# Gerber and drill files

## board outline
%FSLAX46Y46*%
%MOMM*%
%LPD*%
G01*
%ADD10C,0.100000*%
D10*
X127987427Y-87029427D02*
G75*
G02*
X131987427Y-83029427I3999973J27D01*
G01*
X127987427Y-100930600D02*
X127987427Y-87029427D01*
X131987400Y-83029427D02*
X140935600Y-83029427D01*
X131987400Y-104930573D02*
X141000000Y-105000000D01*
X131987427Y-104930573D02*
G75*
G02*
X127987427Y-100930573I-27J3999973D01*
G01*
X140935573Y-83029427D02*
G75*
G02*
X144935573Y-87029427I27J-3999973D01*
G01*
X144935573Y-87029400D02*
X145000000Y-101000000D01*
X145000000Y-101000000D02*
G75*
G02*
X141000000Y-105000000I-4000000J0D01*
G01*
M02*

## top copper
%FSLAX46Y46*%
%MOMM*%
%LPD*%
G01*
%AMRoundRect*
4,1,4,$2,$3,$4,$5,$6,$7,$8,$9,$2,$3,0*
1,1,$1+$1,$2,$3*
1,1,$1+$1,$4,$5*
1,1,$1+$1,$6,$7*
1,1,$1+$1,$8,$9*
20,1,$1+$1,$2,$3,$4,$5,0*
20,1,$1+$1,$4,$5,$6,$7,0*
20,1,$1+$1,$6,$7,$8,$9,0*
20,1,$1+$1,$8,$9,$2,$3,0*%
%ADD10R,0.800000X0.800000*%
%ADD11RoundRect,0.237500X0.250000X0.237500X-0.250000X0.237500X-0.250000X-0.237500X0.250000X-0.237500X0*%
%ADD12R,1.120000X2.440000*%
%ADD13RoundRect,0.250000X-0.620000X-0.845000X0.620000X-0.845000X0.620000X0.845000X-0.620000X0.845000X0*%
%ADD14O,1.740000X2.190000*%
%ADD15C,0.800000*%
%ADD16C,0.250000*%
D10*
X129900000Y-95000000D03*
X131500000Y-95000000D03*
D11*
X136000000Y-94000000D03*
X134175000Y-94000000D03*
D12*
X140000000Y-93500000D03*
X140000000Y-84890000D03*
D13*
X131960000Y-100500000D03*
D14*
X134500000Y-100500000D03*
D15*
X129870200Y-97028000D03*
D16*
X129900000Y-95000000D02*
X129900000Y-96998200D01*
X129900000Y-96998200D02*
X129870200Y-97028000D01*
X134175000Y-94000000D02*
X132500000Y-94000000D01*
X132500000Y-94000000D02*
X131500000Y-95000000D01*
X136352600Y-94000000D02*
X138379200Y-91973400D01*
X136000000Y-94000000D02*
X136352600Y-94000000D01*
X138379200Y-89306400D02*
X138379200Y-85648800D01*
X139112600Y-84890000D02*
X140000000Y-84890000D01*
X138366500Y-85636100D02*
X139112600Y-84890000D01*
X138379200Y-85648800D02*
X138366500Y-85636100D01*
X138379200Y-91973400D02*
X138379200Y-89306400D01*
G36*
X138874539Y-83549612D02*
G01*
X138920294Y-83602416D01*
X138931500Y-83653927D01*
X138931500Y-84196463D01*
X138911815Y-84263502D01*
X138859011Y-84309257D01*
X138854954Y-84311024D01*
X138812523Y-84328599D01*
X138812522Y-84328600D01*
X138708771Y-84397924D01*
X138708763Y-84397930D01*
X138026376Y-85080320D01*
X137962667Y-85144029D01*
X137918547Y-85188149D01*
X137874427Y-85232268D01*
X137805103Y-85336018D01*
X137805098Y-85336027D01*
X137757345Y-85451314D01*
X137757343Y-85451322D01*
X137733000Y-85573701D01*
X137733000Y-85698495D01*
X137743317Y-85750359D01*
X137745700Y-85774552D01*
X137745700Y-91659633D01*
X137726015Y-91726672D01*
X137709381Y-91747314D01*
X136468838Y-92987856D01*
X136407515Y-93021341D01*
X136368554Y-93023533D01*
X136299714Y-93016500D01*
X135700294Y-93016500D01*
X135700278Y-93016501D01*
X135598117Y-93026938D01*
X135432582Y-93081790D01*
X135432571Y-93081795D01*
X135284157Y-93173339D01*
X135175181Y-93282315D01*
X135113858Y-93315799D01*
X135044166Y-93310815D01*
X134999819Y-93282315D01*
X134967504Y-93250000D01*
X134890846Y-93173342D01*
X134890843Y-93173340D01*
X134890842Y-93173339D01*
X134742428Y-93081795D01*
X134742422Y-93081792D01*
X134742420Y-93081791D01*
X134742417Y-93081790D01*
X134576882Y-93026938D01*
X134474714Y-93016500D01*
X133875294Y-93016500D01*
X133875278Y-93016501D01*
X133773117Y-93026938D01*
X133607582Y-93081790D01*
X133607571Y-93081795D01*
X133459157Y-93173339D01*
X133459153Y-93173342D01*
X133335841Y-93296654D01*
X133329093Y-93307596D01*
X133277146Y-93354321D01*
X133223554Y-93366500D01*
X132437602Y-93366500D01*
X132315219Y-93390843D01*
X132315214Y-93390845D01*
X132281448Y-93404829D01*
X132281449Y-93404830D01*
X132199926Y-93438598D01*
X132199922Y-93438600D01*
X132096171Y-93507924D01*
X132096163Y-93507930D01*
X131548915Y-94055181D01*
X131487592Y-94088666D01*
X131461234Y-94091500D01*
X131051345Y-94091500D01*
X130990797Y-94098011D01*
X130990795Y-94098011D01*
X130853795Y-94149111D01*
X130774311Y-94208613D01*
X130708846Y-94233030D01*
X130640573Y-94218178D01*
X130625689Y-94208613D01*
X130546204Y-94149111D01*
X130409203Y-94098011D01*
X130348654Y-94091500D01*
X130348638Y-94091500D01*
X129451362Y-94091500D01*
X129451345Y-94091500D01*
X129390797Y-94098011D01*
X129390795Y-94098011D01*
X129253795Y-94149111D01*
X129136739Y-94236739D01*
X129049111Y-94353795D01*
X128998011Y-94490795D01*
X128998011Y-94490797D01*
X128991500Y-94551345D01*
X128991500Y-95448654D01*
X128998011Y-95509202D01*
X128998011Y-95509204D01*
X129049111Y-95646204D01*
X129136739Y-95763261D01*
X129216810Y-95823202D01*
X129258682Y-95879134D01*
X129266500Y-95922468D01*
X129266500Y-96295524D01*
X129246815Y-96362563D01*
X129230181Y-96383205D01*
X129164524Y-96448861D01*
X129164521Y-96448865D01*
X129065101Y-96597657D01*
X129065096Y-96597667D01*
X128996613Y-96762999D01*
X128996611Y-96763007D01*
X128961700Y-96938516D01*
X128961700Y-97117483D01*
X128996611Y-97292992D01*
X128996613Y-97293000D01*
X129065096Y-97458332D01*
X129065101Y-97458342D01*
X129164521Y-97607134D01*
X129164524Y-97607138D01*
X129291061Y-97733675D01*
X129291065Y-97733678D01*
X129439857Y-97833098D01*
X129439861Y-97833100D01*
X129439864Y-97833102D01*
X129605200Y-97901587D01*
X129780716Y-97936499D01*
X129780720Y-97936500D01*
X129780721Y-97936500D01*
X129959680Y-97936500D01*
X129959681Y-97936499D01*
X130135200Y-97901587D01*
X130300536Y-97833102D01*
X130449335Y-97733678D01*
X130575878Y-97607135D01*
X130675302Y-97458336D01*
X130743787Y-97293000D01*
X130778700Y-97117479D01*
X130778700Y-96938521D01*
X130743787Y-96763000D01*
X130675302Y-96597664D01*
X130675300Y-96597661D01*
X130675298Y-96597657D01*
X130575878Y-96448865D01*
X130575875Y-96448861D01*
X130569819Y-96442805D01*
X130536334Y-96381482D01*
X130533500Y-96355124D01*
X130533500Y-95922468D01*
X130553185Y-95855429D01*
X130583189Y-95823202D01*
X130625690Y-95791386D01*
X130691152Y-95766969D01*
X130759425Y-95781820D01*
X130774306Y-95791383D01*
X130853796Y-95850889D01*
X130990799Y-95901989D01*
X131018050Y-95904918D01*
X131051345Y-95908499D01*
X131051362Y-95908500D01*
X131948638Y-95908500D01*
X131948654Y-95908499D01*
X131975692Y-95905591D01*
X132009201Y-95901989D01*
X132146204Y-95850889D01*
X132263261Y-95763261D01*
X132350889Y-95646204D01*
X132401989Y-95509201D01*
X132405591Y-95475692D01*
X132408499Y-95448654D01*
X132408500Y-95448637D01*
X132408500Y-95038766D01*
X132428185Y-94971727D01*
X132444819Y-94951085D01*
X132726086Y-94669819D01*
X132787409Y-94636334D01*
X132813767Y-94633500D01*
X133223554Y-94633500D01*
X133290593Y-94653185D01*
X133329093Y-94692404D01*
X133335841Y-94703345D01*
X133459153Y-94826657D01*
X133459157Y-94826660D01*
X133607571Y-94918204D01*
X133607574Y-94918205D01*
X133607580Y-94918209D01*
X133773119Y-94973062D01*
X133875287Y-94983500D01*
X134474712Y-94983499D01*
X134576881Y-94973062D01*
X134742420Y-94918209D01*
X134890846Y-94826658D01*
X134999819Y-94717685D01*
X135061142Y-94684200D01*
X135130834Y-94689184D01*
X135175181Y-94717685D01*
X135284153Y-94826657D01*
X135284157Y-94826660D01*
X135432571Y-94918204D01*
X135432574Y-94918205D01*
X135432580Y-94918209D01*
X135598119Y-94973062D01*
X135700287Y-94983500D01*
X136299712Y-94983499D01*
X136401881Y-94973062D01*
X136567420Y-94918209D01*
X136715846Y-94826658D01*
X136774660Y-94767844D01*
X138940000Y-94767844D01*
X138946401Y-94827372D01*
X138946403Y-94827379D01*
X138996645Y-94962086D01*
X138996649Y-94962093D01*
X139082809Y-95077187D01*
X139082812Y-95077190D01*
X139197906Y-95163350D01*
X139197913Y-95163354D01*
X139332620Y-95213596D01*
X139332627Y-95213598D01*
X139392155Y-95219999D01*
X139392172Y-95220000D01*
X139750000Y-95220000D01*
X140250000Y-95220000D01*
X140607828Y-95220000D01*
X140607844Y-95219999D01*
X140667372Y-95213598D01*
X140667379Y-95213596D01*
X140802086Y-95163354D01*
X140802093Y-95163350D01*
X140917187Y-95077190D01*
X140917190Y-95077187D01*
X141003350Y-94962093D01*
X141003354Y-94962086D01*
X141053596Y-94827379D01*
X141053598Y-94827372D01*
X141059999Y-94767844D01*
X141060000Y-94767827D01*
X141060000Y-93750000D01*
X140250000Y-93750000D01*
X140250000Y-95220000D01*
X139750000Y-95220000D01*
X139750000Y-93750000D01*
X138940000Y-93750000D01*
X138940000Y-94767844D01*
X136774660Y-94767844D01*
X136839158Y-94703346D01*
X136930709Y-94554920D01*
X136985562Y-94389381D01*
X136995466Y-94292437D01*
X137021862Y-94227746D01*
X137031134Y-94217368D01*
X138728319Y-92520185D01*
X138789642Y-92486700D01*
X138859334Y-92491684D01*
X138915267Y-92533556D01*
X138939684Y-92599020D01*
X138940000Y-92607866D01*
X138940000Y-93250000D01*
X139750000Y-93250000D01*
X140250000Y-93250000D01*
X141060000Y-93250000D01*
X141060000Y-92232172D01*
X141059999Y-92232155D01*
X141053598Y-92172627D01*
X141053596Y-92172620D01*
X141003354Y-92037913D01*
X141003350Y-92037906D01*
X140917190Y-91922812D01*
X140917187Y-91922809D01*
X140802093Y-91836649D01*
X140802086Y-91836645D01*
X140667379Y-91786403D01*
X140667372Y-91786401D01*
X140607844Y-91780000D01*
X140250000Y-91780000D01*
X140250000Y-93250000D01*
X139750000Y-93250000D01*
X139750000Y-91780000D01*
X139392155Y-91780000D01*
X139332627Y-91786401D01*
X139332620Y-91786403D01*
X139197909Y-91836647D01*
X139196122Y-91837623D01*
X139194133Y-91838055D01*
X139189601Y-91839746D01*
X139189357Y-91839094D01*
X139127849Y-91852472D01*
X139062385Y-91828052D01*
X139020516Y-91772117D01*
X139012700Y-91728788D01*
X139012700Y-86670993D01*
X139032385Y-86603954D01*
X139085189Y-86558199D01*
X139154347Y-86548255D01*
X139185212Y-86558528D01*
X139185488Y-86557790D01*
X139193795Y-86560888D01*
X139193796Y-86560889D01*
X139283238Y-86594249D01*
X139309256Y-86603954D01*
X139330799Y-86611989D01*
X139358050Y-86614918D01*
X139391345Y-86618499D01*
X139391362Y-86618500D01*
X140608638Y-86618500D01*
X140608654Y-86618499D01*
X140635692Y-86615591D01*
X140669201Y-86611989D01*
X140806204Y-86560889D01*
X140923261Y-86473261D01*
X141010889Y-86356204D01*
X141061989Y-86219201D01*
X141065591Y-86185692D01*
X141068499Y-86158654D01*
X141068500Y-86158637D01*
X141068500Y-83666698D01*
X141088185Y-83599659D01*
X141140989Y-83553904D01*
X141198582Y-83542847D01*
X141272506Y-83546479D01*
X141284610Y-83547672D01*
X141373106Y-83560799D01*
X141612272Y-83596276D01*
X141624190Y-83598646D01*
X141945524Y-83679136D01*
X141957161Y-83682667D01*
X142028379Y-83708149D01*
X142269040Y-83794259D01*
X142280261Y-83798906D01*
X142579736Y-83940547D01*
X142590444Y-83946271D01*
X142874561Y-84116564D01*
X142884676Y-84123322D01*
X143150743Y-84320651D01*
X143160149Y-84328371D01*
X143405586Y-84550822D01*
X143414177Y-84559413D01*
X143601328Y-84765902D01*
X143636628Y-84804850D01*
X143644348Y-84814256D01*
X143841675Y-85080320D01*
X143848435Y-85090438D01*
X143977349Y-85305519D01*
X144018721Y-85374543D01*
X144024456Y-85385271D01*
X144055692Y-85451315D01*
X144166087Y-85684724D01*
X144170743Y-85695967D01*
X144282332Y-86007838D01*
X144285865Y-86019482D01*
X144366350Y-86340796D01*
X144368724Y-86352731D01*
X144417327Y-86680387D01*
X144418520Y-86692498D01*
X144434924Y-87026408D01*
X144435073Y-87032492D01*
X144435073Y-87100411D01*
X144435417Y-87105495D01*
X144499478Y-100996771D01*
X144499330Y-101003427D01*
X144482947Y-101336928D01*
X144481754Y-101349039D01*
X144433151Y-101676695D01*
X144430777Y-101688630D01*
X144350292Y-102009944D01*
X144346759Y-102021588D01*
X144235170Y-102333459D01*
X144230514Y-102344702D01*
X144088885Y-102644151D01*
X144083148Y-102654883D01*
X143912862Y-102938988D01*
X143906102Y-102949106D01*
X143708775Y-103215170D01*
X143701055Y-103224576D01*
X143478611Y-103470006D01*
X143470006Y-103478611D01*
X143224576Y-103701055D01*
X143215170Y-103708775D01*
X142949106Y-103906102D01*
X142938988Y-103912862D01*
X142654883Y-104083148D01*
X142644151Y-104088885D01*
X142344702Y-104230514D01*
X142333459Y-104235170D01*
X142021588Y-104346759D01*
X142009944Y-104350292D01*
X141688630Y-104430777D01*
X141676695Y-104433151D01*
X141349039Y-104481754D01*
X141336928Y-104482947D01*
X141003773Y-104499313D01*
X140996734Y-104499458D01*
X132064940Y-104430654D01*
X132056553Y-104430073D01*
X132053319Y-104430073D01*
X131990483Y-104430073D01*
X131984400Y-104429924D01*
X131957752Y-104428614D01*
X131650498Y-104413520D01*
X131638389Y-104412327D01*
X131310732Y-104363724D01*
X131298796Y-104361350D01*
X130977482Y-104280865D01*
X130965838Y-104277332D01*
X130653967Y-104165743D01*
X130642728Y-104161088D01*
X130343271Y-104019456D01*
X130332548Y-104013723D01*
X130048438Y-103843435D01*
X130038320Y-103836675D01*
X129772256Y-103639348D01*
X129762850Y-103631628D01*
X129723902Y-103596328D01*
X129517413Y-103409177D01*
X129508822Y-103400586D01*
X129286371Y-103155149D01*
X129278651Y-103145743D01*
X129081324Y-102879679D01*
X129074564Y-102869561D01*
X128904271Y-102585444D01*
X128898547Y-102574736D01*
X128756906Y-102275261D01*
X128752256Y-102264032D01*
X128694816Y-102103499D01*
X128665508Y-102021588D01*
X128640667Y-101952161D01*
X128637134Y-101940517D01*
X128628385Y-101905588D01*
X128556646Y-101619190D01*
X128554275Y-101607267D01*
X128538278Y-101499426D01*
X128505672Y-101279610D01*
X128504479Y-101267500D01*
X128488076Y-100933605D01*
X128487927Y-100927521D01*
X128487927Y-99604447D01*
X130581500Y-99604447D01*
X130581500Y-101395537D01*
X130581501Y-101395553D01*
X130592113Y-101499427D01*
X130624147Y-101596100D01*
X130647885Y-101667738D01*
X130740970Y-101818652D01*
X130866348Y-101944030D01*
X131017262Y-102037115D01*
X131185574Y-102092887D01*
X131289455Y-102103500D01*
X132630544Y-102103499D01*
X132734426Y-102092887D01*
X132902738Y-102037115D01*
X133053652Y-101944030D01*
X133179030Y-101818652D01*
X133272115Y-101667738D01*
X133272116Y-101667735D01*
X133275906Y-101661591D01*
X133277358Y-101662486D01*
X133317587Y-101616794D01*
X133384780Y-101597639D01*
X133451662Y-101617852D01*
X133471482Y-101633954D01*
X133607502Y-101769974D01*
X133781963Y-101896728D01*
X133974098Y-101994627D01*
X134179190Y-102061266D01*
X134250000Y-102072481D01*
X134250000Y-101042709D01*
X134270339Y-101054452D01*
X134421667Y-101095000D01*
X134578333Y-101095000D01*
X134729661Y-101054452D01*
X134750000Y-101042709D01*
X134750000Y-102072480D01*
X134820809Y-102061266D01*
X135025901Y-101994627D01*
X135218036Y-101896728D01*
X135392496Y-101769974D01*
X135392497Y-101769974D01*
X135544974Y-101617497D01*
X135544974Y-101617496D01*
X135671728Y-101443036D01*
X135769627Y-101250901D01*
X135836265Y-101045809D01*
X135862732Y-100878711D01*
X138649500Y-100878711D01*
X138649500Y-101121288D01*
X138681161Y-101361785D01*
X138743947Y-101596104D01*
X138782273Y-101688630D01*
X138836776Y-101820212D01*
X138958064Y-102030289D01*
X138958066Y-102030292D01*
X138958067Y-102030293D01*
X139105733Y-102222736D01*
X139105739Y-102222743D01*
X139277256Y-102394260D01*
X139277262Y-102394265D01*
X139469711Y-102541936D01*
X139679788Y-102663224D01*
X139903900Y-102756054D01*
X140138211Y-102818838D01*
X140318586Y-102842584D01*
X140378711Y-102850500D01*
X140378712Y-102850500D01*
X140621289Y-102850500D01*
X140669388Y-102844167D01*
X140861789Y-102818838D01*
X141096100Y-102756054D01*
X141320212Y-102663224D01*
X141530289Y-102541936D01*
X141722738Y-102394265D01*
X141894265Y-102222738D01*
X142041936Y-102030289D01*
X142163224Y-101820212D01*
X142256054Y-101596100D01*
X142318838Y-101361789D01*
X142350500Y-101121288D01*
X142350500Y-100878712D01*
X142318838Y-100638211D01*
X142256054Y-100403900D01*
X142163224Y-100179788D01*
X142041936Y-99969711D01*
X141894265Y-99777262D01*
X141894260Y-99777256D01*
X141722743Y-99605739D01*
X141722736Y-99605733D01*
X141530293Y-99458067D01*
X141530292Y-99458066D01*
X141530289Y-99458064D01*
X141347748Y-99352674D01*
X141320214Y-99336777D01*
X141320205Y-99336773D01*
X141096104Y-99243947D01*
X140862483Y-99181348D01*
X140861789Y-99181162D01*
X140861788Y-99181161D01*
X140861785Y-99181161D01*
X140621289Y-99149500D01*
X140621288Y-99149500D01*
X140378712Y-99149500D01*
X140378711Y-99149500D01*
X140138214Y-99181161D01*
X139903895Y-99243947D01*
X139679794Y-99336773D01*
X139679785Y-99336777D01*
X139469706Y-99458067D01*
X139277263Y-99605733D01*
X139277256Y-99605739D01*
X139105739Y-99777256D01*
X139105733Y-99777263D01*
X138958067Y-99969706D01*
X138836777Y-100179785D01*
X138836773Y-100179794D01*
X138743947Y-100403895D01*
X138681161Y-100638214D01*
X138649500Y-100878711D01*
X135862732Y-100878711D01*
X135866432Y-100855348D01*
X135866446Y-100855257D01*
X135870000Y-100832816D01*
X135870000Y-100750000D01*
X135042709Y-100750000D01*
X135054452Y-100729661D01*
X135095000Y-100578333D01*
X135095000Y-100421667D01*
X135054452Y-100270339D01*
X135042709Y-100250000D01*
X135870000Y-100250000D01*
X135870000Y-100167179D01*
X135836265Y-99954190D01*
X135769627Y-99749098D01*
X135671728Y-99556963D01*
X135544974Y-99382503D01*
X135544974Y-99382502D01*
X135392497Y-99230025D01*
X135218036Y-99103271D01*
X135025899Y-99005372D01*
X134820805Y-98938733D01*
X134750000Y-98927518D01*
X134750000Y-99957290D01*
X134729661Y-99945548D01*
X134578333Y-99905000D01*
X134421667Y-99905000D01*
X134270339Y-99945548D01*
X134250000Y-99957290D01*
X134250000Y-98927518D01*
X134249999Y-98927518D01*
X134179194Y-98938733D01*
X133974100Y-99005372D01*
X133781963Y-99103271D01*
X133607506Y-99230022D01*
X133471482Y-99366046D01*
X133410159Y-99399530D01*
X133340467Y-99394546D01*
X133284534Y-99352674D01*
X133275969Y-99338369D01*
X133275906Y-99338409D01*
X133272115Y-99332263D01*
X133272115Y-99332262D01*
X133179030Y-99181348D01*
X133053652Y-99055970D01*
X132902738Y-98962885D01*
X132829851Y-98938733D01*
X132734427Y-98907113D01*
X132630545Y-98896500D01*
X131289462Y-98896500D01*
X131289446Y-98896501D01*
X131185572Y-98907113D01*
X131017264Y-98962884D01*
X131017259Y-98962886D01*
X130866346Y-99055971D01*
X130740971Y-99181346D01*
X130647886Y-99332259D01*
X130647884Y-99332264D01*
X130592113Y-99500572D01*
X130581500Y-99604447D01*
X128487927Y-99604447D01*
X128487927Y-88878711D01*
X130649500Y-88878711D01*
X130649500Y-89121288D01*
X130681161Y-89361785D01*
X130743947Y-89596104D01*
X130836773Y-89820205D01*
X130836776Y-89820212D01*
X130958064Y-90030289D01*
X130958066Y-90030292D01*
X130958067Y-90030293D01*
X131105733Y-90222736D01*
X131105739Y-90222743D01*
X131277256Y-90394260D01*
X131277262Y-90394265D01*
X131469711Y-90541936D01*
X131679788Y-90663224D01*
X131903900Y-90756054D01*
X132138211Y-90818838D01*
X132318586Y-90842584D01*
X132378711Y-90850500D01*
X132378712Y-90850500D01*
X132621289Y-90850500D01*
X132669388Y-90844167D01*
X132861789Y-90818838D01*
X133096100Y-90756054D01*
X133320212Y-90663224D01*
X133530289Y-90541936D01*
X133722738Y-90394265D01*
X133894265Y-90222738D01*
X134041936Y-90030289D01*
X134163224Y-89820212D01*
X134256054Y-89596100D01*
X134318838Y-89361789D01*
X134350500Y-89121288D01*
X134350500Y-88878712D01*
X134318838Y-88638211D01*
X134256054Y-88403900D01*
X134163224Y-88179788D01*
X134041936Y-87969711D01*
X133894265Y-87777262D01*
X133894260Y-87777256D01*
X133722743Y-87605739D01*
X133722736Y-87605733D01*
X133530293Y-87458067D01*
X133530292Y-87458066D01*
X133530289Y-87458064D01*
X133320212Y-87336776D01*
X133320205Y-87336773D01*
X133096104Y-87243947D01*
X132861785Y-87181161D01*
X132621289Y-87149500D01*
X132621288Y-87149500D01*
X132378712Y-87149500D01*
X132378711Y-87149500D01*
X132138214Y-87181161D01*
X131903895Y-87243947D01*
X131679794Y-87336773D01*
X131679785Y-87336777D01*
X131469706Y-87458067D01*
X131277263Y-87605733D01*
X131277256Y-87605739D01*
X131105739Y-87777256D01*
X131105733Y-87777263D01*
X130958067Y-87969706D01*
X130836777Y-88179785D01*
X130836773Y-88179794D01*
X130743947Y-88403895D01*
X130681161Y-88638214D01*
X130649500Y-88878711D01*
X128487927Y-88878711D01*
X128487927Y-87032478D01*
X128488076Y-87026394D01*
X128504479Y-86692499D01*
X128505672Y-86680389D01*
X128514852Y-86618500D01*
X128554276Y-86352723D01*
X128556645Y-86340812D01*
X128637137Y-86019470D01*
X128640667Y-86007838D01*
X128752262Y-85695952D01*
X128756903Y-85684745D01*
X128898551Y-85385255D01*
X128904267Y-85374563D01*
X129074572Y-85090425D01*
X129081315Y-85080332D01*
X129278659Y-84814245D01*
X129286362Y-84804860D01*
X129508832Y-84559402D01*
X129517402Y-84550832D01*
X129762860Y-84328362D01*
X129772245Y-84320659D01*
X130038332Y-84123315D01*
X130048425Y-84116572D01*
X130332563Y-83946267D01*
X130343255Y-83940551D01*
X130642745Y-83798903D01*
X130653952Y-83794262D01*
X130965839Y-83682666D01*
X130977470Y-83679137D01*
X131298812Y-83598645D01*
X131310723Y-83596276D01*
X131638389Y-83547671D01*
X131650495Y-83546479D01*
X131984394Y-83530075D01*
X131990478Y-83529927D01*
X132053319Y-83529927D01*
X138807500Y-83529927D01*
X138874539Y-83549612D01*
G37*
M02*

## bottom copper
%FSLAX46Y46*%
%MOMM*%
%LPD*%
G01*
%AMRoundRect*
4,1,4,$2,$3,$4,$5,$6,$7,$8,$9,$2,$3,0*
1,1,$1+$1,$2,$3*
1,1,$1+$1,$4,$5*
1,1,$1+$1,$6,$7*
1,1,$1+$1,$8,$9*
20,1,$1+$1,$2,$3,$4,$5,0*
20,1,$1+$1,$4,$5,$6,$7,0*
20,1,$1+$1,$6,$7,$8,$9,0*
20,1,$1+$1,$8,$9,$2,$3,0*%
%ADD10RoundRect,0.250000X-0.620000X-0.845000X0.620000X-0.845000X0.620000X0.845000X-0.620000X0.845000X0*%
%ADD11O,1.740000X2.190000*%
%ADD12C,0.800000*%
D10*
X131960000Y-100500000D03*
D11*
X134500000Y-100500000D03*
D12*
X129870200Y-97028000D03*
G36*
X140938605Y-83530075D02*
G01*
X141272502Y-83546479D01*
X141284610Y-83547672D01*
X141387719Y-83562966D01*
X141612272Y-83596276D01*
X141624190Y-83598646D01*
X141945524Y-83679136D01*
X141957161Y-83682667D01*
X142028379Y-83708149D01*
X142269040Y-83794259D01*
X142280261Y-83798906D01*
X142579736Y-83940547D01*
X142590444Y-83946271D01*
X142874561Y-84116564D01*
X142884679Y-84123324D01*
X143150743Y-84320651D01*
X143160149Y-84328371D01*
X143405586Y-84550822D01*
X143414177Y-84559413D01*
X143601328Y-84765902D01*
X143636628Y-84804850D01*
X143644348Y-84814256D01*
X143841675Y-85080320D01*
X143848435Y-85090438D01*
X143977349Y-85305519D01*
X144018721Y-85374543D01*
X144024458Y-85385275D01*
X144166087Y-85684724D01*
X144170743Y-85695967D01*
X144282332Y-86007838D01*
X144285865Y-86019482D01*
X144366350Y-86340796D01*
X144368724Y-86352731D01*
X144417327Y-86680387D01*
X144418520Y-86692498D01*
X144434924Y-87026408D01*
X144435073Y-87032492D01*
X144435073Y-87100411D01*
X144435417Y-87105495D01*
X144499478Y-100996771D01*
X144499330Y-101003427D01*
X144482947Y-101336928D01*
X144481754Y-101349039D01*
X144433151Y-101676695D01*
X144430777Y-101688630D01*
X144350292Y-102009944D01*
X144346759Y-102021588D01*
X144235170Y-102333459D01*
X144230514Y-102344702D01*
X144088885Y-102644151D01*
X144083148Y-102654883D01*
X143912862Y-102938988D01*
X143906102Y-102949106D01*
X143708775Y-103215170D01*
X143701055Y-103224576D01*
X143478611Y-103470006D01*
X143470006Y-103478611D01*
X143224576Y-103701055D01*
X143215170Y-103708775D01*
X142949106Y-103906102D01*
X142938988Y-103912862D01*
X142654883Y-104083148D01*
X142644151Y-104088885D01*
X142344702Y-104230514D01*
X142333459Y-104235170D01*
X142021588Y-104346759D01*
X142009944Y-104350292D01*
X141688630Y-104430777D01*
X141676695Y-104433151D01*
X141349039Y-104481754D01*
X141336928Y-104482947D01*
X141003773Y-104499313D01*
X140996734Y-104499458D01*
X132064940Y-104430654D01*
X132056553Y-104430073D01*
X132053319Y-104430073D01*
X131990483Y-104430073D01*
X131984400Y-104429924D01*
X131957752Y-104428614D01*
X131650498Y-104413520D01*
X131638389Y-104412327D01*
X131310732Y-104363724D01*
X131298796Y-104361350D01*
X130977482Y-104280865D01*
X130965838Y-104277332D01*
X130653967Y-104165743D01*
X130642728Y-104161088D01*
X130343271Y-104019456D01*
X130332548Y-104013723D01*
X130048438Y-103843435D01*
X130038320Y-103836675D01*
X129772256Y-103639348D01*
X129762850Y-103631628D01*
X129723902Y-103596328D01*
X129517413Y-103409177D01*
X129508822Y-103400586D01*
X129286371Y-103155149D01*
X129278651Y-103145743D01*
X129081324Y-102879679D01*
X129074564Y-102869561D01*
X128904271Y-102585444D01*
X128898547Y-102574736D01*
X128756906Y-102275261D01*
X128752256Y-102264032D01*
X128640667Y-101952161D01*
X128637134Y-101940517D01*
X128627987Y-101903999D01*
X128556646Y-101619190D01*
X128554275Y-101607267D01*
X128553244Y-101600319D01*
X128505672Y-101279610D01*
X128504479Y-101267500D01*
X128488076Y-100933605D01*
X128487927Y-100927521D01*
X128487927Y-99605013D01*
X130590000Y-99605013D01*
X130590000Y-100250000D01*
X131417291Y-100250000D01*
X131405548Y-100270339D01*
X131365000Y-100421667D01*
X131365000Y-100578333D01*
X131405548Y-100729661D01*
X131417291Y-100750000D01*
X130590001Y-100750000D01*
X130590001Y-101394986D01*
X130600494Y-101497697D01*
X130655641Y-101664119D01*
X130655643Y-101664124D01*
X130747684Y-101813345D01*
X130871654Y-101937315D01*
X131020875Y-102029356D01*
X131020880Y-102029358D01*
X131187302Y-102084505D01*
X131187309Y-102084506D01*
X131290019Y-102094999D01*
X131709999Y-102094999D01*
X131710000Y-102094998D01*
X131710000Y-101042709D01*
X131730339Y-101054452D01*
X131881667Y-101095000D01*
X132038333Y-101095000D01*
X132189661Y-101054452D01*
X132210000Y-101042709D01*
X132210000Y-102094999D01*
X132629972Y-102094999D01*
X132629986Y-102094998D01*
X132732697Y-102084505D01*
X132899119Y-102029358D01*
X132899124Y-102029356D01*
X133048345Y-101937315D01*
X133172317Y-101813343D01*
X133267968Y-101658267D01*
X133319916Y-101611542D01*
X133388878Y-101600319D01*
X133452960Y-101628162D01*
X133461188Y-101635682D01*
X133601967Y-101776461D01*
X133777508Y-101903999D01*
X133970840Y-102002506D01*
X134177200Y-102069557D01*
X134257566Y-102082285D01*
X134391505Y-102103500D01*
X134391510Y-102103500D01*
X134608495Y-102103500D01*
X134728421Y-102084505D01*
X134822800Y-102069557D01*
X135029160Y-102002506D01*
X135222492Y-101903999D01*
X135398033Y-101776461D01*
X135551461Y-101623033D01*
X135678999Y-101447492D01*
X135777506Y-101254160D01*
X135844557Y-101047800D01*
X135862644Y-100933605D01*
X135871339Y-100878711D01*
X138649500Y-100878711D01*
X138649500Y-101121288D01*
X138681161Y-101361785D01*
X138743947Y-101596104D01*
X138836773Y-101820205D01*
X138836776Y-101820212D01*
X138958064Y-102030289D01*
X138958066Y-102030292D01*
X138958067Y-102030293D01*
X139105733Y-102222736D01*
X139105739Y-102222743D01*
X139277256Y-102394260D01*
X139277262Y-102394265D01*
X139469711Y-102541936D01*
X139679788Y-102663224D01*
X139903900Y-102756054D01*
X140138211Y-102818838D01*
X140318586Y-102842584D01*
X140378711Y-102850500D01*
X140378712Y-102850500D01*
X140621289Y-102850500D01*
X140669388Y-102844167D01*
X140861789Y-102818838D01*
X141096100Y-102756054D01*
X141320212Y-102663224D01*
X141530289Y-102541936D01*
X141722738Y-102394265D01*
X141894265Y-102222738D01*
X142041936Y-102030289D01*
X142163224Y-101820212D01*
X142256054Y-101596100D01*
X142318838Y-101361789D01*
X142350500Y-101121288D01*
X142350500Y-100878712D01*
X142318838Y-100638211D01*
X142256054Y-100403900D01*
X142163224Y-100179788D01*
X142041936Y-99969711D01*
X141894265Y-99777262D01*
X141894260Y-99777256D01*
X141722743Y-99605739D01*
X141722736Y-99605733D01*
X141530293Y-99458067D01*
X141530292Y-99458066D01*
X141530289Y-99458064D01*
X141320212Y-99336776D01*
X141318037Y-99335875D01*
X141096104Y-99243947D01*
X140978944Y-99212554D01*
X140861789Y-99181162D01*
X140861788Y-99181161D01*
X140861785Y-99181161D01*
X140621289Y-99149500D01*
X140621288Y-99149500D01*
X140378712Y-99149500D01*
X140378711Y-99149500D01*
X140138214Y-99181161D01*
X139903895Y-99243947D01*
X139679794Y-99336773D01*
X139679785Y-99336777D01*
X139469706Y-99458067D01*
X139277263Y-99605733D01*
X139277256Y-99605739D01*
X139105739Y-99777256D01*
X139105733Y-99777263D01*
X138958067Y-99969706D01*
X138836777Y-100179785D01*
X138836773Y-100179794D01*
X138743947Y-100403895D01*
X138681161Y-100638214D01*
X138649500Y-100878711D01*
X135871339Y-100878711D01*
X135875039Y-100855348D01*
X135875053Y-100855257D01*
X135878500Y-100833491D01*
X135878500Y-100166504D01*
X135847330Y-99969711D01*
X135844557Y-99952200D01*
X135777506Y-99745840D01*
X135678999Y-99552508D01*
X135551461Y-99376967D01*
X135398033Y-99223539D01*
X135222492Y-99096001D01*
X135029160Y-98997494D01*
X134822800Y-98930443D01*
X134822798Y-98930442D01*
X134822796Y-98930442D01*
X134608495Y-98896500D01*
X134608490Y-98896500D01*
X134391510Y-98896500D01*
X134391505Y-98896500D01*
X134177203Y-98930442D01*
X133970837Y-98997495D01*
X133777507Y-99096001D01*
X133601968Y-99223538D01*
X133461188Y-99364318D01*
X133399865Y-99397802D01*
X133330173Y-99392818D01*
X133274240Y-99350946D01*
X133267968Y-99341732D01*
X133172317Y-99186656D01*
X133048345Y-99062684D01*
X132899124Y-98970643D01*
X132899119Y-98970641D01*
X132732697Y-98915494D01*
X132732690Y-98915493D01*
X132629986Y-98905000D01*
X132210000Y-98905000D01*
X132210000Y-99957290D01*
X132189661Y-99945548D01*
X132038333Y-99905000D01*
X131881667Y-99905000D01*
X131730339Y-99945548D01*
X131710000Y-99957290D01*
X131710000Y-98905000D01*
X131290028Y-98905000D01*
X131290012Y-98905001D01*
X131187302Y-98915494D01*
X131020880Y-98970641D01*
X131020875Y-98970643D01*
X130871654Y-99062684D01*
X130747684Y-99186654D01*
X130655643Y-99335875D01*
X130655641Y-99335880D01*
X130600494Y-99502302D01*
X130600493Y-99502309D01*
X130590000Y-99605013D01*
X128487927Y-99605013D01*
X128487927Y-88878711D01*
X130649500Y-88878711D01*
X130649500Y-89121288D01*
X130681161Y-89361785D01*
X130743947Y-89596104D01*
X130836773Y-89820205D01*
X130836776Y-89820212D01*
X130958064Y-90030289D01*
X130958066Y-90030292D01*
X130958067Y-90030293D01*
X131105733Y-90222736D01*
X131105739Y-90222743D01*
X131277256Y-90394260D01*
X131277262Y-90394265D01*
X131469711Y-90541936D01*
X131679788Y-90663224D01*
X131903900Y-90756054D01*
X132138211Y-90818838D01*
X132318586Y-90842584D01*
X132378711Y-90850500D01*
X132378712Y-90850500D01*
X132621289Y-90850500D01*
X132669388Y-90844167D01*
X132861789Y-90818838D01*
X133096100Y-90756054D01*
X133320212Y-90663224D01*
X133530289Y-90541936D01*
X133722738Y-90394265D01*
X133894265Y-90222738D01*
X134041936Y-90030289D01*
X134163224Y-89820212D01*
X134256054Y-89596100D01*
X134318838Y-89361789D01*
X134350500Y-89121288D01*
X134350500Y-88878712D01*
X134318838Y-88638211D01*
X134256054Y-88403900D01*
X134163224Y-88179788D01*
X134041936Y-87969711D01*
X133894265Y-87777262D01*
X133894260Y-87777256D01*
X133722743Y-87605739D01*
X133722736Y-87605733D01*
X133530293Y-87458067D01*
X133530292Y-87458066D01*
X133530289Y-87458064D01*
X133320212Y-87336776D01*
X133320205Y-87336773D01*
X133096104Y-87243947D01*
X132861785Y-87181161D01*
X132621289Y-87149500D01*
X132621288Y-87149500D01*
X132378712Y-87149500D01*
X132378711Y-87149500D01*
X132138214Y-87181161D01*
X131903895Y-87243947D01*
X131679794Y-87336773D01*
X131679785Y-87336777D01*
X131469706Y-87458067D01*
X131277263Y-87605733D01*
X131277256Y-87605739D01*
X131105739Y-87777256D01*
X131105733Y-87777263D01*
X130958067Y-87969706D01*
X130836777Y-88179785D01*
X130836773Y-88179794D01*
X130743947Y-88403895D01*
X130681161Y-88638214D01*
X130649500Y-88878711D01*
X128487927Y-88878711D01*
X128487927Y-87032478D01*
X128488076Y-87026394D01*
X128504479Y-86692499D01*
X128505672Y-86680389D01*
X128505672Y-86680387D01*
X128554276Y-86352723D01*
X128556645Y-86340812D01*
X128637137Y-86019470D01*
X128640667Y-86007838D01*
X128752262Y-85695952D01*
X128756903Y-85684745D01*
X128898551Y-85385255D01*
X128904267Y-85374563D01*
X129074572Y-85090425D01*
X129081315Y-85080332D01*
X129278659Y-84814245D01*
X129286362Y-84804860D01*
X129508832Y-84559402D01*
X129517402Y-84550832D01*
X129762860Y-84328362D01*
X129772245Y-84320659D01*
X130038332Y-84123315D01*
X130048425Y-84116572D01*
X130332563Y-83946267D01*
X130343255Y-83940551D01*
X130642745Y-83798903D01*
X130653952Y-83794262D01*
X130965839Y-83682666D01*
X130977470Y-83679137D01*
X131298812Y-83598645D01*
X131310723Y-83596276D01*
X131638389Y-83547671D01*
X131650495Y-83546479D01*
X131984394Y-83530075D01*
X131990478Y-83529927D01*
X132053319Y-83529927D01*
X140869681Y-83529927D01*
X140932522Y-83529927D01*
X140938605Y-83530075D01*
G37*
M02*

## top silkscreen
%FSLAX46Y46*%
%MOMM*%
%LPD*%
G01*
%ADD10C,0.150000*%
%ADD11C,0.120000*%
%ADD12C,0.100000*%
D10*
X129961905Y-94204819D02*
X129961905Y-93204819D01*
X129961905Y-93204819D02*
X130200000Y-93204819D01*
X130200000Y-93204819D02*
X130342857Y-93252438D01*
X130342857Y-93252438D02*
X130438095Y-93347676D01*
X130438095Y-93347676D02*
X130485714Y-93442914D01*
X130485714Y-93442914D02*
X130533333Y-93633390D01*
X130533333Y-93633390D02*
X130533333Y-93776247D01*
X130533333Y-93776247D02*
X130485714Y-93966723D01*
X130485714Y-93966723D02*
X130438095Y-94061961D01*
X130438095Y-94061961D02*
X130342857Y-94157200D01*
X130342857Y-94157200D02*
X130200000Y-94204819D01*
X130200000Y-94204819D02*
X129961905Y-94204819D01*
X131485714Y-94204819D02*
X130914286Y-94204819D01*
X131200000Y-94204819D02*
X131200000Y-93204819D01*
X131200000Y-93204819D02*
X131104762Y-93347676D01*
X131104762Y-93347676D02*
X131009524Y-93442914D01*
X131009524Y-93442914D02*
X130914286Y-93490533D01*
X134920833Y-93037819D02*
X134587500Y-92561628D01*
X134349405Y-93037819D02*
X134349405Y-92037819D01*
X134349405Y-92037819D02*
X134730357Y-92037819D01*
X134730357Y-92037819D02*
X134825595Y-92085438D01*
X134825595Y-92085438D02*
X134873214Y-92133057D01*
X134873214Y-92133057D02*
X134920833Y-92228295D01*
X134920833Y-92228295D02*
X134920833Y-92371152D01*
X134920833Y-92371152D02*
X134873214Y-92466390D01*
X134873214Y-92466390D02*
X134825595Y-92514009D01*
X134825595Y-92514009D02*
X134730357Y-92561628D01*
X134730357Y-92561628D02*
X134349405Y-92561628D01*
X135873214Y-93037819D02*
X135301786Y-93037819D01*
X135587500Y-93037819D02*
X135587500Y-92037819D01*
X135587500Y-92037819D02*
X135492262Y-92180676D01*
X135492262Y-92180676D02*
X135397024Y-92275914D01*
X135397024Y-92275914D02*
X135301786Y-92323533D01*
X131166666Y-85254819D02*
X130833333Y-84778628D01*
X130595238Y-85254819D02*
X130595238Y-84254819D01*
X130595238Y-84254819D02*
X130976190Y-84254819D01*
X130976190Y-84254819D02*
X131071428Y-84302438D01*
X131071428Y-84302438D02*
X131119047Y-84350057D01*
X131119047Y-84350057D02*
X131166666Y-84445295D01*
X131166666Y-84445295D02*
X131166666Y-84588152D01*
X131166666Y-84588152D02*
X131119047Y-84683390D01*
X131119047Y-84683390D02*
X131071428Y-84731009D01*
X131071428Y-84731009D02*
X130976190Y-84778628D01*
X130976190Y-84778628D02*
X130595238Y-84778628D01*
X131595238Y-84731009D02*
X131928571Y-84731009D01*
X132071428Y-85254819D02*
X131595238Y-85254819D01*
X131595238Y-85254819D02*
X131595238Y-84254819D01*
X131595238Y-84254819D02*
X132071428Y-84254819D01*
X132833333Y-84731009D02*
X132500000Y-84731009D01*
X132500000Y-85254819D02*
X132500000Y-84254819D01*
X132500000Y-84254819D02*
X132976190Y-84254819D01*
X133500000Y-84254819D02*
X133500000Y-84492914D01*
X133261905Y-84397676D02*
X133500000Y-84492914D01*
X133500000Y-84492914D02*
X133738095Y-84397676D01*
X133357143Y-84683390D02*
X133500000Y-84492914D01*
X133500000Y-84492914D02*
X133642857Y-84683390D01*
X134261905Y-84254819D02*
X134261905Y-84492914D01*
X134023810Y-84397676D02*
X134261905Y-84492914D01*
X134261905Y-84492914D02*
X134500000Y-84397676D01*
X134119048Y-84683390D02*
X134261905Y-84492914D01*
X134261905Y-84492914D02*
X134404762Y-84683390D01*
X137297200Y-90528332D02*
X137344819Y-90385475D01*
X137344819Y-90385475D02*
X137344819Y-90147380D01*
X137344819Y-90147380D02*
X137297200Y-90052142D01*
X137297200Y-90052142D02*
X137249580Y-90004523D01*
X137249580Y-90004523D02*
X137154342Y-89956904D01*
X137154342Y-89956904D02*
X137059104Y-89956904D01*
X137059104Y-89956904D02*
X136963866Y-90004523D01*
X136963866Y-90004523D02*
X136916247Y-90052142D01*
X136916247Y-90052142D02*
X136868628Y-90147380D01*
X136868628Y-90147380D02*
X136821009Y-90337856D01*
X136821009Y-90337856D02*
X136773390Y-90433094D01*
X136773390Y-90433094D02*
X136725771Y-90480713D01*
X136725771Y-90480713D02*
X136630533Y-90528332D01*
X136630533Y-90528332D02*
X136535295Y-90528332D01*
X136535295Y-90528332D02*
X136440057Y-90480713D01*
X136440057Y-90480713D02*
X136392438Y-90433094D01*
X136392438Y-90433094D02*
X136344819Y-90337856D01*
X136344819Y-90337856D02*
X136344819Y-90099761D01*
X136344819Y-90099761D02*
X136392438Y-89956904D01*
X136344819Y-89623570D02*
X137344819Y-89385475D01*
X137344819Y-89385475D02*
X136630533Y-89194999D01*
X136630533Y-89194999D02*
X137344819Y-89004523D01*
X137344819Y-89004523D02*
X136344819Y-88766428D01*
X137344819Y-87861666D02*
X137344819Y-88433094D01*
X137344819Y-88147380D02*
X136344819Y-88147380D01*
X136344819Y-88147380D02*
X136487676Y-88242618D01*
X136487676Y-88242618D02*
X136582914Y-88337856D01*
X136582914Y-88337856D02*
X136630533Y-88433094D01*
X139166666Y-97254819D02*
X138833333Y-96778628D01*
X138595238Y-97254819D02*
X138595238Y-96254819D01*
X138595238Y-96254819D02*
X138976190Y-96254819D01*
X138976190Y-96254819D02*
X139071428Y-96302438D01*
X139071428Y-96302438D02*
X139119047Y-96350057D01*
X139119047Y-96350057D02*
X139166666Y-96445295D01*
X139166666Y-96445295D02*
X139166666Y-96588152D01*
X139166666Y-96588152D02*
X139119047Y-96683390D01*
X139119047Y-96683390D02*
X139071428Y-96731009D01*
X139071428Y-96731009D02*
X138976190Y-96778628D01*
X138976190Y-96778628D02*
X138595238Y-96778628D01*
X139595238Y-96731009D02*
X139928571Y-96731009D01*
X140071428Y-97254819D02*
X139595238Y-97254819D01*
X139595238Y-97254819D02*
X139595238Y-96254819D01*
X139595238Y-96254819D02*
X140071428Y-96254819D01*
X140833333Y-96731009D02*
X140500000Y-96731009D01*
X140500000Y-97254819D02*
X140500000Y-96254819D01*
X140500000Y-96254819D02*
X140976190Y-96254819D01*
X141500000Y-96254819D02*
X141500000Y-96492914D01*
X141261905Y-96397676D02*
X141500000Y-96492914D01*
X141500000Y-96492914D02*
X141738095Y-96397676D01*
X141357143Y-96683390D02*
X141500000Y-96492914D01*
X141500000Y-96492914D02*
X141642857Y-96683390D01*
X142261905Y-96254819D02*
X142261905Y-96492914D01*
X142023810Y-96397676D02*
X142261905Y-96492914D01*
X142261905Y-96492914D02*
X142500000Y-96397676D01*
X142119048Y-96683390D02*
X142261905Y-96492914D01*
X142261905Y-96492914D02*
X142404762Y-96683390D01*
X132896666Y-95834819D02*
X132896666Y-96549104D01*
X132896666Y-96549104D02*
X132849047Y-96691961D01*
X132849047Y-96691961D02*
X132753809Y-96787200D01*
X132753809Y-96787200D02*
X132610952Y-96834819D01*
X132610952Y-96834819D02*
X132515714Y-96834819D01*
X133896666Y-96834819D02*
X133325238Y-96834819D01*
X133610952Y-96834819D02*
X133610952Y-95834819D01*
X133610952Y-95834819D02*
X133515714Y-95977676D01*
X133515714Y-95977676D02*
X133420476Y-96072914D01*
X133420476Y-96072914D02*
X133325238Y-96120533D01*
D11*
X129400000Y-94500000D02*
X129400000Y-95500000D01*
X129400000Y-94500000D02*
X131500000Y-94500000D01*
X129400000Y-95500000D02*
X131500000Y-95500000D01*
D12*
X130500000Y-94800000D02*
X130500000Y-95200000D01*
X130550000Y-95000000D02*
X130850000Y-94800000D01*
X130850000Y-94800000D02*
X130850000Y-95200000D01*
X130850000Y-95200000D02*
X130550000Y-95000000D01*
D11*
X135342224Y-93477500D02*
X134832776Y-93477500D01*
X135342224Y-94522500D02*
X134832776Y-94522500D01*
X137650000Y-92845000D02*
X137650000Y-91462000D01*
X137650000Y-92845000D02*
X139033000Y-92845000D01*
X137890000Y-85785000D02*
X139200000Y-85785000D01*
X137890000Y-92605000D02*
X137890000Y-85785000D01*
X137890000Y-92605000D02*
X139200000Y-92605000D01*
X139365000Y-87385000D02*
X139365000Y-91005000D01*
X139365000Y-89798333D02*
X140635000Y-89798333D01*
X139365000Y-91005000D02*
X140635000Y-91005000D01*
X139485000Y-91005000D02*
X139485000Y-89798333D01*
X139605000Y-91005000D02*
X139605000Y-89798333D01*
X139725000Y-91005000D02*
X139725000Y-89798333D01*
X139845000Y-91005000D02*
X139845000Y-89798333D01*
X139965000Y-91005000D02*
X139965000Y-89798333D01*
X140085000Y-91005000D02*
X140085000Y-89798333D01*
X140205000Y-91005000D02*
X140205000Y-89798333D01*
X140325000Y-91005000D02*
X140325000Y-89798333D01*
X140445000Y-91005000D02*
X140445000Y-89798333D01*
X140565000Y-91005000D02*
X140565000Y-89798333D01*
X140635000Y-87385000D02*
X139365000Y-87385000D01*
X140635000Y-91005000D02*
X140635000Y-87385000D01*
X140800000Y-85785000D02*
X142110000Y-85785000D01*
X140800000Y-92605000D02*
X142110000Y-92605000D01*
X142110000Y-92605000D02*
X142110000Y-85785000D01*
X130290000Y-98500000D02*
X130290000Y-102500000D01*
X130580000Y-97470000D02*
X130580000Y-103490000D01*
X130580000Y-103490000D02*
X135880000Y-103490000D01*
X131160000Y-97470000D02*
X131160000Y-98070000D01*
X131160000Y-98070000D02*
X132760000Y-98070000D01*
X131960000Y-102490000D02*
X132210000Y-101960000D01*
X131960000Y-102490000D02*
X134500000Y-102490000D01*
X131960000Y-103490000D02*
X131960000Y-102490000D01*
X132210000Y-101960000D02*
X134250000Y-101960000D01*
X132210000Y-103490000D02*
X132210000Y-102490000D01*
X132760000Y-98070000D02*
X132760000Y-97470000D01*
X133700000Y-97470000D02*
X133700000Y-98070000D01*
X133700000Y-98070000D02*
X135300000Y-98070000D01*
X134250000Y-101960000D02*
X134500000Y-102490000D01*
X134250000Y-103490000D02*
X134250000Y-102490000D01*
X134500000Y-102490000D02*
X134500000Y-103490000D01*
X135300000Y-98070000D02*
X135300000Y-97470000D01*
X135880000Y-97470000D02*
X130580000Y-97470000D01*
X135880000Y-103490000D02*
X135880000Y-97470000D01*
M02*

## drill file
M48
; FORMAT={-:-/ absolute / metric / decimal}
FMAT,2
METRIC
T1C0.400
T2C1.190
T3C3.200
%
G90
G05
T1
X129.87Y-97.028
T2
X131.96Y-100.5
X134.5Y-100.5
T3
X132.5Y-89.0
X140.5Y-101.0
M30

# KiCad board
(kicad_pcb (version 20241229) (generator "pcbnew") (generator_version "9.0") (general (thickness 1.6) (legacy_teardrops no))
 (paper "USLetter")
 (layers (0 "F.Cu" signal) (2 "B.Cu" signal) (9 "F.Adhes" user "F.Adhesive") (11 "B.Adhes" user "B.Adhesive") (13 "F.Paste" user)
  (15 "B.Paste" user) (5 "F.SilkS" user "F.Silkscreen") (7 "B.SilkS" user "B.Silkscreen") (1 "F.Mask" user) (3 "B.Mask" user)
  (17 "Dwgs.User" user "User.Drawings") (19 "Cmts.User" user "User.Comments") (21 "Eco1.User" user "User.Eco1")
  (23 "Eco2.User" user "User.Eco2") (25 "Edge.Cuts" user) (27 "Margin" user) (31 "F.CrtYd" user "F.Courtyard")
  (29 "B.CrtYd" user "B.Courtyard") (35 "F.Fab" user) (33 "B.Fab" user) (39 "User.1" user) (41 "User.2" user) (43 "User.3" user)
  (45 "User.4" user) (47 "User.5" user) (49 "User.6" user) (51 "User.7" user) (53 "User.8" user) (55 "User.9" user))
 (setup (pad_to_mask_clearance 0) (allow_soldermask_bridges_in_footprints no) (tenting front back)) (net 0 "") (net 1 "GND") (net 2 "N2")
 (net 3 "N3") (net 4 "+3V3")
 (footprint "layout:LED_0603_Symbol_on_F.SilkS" (layer "F.Cu") (at 130.7 95)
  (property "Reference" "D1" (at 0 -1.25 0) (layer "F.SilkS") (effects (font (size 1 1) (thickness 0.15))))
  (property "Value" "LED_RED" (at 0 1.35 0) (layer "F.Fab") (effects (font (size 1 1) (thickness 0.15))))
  (fp_line (start -1.3 -0.5) (end -1.3 0.5) (stroke (width 0.12) (type solid)) (layer "F.SilkS"))
  (fp_line (start -1.3 -0.5) (end 0.8 -0.5) (stroke (width 0.12) (type solid)) (layer "F.SilkS"))
  (fp_line (start -1.3 0.5) (end 0.8 0.5) (stroke (width 0.12) (type solid)) (layer "F.SilkS"))
  (fp_line (start -0.2 -0.2) (end -0.2 0.2) (stroke (width 0.1) (type solid)) (layer "F.SilkS"))
  (fp_line (start -0.15 0) (end 0.15 -0.2) (stroke (width 0.1) (type solid)) (layer "F.SilkS"))
  (fp_line (start 0.15 -0.2) (end 0.15 0.2) (stroke (width 0.1) (type solid)) (layer "F.SilkS"))
  (fp_line (start 0.15 0.2) (end -0.15 0) (stroke (width 0.1) (type solid)) (layer "F.SilkS"))
  (pad "1" smd rect (at -0.8 0 180) (size 0.8 0.8) (layers "F.Cu" "F.Mask" "F.Paste") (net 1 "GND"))
  (pad "2" smd rect (at 0.8 0 180) (size 0.8 0.8) (layers "F.Cu" "F.Mask" "F.Paste") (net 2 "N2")))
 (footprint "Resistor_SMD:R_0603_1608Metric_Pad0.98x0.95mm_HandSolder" (layer "F.Cu") (at 135.0875 94 180)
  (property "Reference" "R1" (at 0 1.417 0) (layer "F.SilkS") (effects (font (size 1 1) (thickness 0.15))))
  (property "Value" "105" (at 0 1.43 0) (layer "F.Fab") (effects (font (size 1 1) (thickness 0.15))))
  (fp_line (start -0.254724 0.5225) (end 0.254724 0.5225) (stroke (width 0.12) (type solid)) (layer "F.SilkS"))
  (fp_line (start -0.254724 -0.5225) (end 0.254724 -0.5225) (stroke (width 0.12) (type solid)) (layer "F.SilkS"))
  (pad "1" smd roundrect (at -0.9125 0 180) (size 0.975 0.95) (layers "F.Cu" "F.Mask" "F.Paste") (roundrect_rratio 0.25) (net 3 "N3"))
  (pad "2" smd roundrect (at 0.9125 0 180) (size 0.975 0.95) (layers "F.Cu" "F.Mask" "F.Paste") (roundrect_rratio 0.25) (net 2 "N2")))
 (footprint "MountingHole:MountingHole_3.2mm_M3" (layer "F.Cu") (at 132.5 89)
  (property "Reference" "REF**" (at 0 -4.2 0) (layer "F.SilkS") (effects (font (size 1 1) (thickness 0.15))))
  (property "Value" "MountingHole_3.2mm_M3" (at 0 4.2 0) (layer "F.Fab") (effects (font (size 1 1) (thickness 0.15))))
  (pad "" np_thru_hole circle (at 0 0) (size 3.2 3.2) (drill 3.2) (layers "*.Cu" "*.Mask")))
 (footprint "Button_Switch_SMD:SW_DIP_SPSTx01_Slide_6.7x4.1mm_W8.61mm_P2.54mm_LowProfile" (layer "F.Cu") (at 140 89.195 90)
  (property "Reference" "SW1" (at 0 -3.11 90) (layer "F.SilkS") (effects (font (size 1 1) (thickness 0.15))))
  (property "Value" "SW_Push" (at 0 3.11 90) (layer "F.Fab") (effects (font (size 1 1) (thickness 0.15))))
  (fp_line (start -3.65 -2.35) (end -2.267 -2.35) (stroke (width 0.12) (type solid)) (layer "F.SilkS"))
  (fp_line (start -3.65 -2.35) (end -3.65 -0.967) (stroke (width 0.12) (type solid)) (layer "F.SilkS"))
  (fp_line (start 3.41 -2.11) (end 3.41 -0.8) (stroke (width 0.12) (type solid)) (layer "F.SilkS"))
  (fp_line (start -3.41 -2.11) (end 3.41 -2.11) (stroke (width 0.12) (type solid)) (layer "F.SilkS"))
  (fp_line (start -3.41 -2.11) (end -3.41 -0.8) (stroke (width 0.12) (type solid)) (layer "F.SilkS"))
  (fp_line (start 1.81 -0.635) (end -1.81 -0.635) (stroke (width 0.12) (type solid)) (layer "F.SilkS"))
  (fp_line (start -0.603333 -0.635) (end -0.603333 0.635) (stroke (width 0.12) (type solid)) (layer "F.SilkS"))
  (fp_line (start -1.81 -0.635) (end -1.81 0.635) (stroke (width 0.12) (type solid)) (layer "F.SilkS"))
  (fp_line (start -1.81 -0.515) (end -0.603333 -0.515) (stroke (width 0.12) (type solid)) (layer "F.SilkS"))
  (fp_line (start -1.81 -0.395) (end -0.603333 -0.395) (stroke (width 0.12) (type solid)) (layer "F.SilkS"))
  (fp_line (start -1.81 -0.275) (end -0.603333 -0.275) (stroke (width 0.12) (type solid)) (layer "F.SilkS"))
  (fp_line (start -1.81 -0.155) (end -0.603333 -0.155) (stroke (width 0.12) (type solid)) (layer "F.SilkS"))
  (fp_line (start -1.81 -0.035) (end -0.603333 -0.035) (stroke (width 0.12) (type solid)) (layer "F.SilkS"))
  (fp_line (start -1.81 0.085) (end -0.603333 0.085) (stroke (width 0.12) (type solid)) (layer "F.SilkS"))
  (fp_line (start -1.81 0.205) (end -0.603333 0.205) (stroke (width 0.12) (type solid)) (layer "F.SilkS"))
  (fp_line (start -1.81 0.325) (end -0.603333 0.325) (stroke (width 0.12) (type solid)) (layer "F.SilkS"))
  (fp_line (start -1.81 0.445) (end -0.603333 0.445) (stroke (width 0.12) (type solid)) (layer "F.SilkS"))
  (fp_line (start -1.81 0.565) (end -0.603333 0.565) (stroke (width 0.12) (type solid)) (layer "F.SilkS"))
  (fp_line (start 1.81 0.635) (end 1.81 -0.635) (stroke (width 0.12) (type solid)) (layer "F.SilkS"))
  (fp_line (start -1.81 0.635) (end 1.81 0.635) (stroke (width 0.12) (type solid)) (layer "F.SilkS"))
  (fp_line (start 3.41 0.8) (end 3.41 2.11) (stroke (width 0.12) (type solid)) (layer "F.SilkS"))
  (fp_line (start -3.41 0.8) (end -3.41 2.11) (stroke (width 0.12) (type solid)) (layer "F.SilkS"))
  (fp_line (start -3.41 2.11) (end 3.41 2.11) (stroke (width 0.12) (type solid)) (layer "F.SilkS"))
  (pad "1" smd rect (at -4.305 0 90) (size 2.44 1.12) (layers "F.Cu" "F.Mask" "F.Paste") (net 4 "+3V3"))
  (pad "2" smd rect (at 4.305 0 90) (size 2.44 1.12) (layers "F.Cu" "F.Mask" "F.Paste") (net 3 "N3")))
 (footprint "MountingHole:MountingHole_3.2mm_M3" (layer "F.Cu") (at 140.5 101)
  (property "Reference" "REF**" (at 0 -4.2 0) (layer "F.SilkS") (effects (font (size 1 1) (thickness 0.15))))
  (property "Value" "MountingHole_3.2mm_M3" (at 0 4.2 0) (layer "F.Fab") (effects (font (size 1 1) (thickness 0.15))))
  (pad "" np_thru_hole circle (at 0 0) (size 3.2 3.2) (drill 3.2) (layers "*.Cu" "*.Mask")))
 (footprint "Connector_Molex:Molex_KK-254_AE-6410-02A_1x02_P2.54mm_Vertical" (layer "F.Cu") (at 131.96 100.5)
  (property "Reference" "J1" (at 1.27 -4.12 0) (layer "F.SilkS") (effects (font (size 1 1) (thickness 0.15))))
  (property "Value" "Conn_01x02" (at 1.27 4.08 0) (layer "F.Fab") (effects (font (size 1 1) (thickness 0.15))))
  (fp_line (start -1.67 -2) (end -1.67 2) (stroke (width 0.12) (type solid)) (layer "F.SilkS"))
  (fp_line (start -1.38 -3.03) (end -1.38 2.99) (stroke (width 0.12) (type solid)) (layer "F.SilkS"))
  (fp_line (start -1.38 2.99) (end 3.92 2.99) (stroke (width 0.12) (type solid)) (layer "F.SilkS"))
  (fp_line (start -0.8 -3.03) (end -0.8 -2.43) (stroke (width 0.12) (type solid)) (layer "F.SilkS"))
  (fp_line (start -0.8 -2.43) (end 0.8 -2.43) (stroke (width 0.12) (type solid)) (layer "F.SilkS"))
  (fp_line (start 0 1.99) (end 0.25 1.46) (stroke (width 0.12) (type solid)) (layer "F.SilkS"))
  (fp_line (start 0 1.99) (end 2.54 1.99) (stroke (width 0.12) (type solid)) (layer "F.SilkS"))
  (fp_line (start 0 2.99) (end 0 1.99) (stroke (width 0.12) (type solid)) (layer "F.SilkS"))
  (fp_line (start 0.25 1.46) (end 2.29 1.46) (stroke (width 0.12) (type solid)) (layer "F.SilkS"))
  (fp_line (start 0.25 2.99) (end 0.25 1.99) (stroke (width 0.12) (type solid)) (layer "F.SilkS"))
  (fp_line (start 0.8 -2.43) (end 0.8 -3.03) (stroke (width 0.12) (type solid)) (layer "F.SilkS"))
  (fp_line (start 1.74 -3.03) (end 1.74 -2.43) (stroke (width 0.12) (type solid)) (layer "F.SilkS"))
  (fp_line (start 1.74 -2.43) (end 3.34 -2.43) (stroke (width 0.12) (type solid)) (layer "F.SilkS"))
  (fp_line (start 2.29 1.46) (end 2.54 1.99) (stroke (width 0.12) (type solid)) (layer "F.SilkS"))
  (fp_line (start 2.29 2.99) (end 2.29 1.99) (stroke (width 0.12) (type solid)) (layer "F.SilkS"))
  (fp_line (start 2.54 1.99) (end 2.54 2.99) (stroke (width 0.12) (type solid)) (layer "F.SilkS"))
  (fp_line (start 3.34 -2.43) (end 3.34 -3.03) (stroke (width 0.12) (type solid)) (layer "F.SilkS"))
  (fp_line (start 3.92 -3.03) (end -1.38 -3.03) (stroke (width 0.12) (type solid)) (layer "F.SilkS"))
  (fp_line (start 3.92 2.99) (end 3.92 -3.03) (stroke (width 0.12) (type solid)) (layer "F.SilkS"))
  (pad "1" thru_hole roundrect (at 0 0) (size 1.74 2.19) (drill 1.19) (layers "*.Cu" "*.Mask") (remove_unused_layers no)
   (roundrect_rratio 0.143678) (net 1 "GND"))
  (pad "2" thru_hole oval (at 2.54 0) (size 1.74 2.19) (drill 1.19) (layers "*.Cu" "*.Mask") (remove_unused_layers no) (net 4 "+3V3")))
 (gr_arc (start 127.987427 87.029427) (mid 129.159 84.201) (end 131.987427 83.029427) (stroke (width 0.1) (type default))
  (layer "Edge.Cuts"))
 (gr_line (start 127.987427 100.9306) (end 127.987427 87.029427) (stroke (width 0.1) (type default)) (layer "Edge.Cuts"))
 (gr_line (start 131.9874 83.029427) (end 140.9356 83.029427) (stroke (width 0.1) (type default)) (layer "Edge.Cuts"))
 (gr_line (start 131.9874 104.930573) (end 141 105) (stroke (width 0.1) (type default)) (layer "Edge.Cuts"))
 (gr_arc (start 131.987427 104.930573) (mid 129.159 103.759) (end 127.987427 100.930573) (stroke (width 0.1) (type default))
  (layer "Edge.Cuts"))
 (gr_arc (start 140.935573 83.029427) (mid 143.764 84.201) (end 144.935573 87.029427) (stroke (width 0.1) (type default))
  (layer "Edge.Cuts"))
 (gr_line (start 144.935573 87.0294) (end 145 101) (stroke (width 0.1) (type default)) (layer "Edge.Cuts"))
 (gr_arc (start 145 101) (mid 143.828427 103.828427) (end 141 105) (stroke (width 0.1) (type default)) (layer "Edge.Cuts"))
 (segment (start 129.9 95) (end 129.9 96.9982) (width 0.25) (layer "F.Cu") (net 1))
 (segment (start 129.9 96.9982) (end 129.8702 97.028) (width 0.25) (layer "F.Cu") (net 1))
 (via (at 129.8702 97.028) (size 0.8) (drill 0.4) (layers "F.Cu" "B.Cu") (free yes) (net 1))
 (segment (start 134.175 94) (end 132.5 94) (width 0.25) (layer "F.Cu") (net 2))
 (segment (start 132.5 94) (end 131.5 95) (width 0.25) (layer "F.Cu") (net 2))
 (segment (start 136.3526 94) (end 138.3792 91.9734) (width 0.25) (layer "F.Cu") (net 3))
 (segment (start 136 94) (end 136.3526 94) (width 0.25) (layer "F.Cu") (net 3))
 (segment (start 138.3792 89.3064) (end 138.3792 85.6488) (width 0.25) (layer "F.Cu") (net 3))
 (segment (start 139.1126 84.89) (end 140 84.89) (width 0.25) (layer "F.Cu") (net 3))
 (segment (start 138.3665 85.6361) (end 139.1126 84.89) (width 0.25) (layer "F.Cu") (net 3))
 (segment (start 138.3792 85.6488) (end 138.3665 85.6361) (width 0.25) (layer "F.Cu") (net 3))
 (segment (start 138.3792 91.9734) (end 138.3792 89.3064) (width 0.25) (layer "F.Cu") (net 3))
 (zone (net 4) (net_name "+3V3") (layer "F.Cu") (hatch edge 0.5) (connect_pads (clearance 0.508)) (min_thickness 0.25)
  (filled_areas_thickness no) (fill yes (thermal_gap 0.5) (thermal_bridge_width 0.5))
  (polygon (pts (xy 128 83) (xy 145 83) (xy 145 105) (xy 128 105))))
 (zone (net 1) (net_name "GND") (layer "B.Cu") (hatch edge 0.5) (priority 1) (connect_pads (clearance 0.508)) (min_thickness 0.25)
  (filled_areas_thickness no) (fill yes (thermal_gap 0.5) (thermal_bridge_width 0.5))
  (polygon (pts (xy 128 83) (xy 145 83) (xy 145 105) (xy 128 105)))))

